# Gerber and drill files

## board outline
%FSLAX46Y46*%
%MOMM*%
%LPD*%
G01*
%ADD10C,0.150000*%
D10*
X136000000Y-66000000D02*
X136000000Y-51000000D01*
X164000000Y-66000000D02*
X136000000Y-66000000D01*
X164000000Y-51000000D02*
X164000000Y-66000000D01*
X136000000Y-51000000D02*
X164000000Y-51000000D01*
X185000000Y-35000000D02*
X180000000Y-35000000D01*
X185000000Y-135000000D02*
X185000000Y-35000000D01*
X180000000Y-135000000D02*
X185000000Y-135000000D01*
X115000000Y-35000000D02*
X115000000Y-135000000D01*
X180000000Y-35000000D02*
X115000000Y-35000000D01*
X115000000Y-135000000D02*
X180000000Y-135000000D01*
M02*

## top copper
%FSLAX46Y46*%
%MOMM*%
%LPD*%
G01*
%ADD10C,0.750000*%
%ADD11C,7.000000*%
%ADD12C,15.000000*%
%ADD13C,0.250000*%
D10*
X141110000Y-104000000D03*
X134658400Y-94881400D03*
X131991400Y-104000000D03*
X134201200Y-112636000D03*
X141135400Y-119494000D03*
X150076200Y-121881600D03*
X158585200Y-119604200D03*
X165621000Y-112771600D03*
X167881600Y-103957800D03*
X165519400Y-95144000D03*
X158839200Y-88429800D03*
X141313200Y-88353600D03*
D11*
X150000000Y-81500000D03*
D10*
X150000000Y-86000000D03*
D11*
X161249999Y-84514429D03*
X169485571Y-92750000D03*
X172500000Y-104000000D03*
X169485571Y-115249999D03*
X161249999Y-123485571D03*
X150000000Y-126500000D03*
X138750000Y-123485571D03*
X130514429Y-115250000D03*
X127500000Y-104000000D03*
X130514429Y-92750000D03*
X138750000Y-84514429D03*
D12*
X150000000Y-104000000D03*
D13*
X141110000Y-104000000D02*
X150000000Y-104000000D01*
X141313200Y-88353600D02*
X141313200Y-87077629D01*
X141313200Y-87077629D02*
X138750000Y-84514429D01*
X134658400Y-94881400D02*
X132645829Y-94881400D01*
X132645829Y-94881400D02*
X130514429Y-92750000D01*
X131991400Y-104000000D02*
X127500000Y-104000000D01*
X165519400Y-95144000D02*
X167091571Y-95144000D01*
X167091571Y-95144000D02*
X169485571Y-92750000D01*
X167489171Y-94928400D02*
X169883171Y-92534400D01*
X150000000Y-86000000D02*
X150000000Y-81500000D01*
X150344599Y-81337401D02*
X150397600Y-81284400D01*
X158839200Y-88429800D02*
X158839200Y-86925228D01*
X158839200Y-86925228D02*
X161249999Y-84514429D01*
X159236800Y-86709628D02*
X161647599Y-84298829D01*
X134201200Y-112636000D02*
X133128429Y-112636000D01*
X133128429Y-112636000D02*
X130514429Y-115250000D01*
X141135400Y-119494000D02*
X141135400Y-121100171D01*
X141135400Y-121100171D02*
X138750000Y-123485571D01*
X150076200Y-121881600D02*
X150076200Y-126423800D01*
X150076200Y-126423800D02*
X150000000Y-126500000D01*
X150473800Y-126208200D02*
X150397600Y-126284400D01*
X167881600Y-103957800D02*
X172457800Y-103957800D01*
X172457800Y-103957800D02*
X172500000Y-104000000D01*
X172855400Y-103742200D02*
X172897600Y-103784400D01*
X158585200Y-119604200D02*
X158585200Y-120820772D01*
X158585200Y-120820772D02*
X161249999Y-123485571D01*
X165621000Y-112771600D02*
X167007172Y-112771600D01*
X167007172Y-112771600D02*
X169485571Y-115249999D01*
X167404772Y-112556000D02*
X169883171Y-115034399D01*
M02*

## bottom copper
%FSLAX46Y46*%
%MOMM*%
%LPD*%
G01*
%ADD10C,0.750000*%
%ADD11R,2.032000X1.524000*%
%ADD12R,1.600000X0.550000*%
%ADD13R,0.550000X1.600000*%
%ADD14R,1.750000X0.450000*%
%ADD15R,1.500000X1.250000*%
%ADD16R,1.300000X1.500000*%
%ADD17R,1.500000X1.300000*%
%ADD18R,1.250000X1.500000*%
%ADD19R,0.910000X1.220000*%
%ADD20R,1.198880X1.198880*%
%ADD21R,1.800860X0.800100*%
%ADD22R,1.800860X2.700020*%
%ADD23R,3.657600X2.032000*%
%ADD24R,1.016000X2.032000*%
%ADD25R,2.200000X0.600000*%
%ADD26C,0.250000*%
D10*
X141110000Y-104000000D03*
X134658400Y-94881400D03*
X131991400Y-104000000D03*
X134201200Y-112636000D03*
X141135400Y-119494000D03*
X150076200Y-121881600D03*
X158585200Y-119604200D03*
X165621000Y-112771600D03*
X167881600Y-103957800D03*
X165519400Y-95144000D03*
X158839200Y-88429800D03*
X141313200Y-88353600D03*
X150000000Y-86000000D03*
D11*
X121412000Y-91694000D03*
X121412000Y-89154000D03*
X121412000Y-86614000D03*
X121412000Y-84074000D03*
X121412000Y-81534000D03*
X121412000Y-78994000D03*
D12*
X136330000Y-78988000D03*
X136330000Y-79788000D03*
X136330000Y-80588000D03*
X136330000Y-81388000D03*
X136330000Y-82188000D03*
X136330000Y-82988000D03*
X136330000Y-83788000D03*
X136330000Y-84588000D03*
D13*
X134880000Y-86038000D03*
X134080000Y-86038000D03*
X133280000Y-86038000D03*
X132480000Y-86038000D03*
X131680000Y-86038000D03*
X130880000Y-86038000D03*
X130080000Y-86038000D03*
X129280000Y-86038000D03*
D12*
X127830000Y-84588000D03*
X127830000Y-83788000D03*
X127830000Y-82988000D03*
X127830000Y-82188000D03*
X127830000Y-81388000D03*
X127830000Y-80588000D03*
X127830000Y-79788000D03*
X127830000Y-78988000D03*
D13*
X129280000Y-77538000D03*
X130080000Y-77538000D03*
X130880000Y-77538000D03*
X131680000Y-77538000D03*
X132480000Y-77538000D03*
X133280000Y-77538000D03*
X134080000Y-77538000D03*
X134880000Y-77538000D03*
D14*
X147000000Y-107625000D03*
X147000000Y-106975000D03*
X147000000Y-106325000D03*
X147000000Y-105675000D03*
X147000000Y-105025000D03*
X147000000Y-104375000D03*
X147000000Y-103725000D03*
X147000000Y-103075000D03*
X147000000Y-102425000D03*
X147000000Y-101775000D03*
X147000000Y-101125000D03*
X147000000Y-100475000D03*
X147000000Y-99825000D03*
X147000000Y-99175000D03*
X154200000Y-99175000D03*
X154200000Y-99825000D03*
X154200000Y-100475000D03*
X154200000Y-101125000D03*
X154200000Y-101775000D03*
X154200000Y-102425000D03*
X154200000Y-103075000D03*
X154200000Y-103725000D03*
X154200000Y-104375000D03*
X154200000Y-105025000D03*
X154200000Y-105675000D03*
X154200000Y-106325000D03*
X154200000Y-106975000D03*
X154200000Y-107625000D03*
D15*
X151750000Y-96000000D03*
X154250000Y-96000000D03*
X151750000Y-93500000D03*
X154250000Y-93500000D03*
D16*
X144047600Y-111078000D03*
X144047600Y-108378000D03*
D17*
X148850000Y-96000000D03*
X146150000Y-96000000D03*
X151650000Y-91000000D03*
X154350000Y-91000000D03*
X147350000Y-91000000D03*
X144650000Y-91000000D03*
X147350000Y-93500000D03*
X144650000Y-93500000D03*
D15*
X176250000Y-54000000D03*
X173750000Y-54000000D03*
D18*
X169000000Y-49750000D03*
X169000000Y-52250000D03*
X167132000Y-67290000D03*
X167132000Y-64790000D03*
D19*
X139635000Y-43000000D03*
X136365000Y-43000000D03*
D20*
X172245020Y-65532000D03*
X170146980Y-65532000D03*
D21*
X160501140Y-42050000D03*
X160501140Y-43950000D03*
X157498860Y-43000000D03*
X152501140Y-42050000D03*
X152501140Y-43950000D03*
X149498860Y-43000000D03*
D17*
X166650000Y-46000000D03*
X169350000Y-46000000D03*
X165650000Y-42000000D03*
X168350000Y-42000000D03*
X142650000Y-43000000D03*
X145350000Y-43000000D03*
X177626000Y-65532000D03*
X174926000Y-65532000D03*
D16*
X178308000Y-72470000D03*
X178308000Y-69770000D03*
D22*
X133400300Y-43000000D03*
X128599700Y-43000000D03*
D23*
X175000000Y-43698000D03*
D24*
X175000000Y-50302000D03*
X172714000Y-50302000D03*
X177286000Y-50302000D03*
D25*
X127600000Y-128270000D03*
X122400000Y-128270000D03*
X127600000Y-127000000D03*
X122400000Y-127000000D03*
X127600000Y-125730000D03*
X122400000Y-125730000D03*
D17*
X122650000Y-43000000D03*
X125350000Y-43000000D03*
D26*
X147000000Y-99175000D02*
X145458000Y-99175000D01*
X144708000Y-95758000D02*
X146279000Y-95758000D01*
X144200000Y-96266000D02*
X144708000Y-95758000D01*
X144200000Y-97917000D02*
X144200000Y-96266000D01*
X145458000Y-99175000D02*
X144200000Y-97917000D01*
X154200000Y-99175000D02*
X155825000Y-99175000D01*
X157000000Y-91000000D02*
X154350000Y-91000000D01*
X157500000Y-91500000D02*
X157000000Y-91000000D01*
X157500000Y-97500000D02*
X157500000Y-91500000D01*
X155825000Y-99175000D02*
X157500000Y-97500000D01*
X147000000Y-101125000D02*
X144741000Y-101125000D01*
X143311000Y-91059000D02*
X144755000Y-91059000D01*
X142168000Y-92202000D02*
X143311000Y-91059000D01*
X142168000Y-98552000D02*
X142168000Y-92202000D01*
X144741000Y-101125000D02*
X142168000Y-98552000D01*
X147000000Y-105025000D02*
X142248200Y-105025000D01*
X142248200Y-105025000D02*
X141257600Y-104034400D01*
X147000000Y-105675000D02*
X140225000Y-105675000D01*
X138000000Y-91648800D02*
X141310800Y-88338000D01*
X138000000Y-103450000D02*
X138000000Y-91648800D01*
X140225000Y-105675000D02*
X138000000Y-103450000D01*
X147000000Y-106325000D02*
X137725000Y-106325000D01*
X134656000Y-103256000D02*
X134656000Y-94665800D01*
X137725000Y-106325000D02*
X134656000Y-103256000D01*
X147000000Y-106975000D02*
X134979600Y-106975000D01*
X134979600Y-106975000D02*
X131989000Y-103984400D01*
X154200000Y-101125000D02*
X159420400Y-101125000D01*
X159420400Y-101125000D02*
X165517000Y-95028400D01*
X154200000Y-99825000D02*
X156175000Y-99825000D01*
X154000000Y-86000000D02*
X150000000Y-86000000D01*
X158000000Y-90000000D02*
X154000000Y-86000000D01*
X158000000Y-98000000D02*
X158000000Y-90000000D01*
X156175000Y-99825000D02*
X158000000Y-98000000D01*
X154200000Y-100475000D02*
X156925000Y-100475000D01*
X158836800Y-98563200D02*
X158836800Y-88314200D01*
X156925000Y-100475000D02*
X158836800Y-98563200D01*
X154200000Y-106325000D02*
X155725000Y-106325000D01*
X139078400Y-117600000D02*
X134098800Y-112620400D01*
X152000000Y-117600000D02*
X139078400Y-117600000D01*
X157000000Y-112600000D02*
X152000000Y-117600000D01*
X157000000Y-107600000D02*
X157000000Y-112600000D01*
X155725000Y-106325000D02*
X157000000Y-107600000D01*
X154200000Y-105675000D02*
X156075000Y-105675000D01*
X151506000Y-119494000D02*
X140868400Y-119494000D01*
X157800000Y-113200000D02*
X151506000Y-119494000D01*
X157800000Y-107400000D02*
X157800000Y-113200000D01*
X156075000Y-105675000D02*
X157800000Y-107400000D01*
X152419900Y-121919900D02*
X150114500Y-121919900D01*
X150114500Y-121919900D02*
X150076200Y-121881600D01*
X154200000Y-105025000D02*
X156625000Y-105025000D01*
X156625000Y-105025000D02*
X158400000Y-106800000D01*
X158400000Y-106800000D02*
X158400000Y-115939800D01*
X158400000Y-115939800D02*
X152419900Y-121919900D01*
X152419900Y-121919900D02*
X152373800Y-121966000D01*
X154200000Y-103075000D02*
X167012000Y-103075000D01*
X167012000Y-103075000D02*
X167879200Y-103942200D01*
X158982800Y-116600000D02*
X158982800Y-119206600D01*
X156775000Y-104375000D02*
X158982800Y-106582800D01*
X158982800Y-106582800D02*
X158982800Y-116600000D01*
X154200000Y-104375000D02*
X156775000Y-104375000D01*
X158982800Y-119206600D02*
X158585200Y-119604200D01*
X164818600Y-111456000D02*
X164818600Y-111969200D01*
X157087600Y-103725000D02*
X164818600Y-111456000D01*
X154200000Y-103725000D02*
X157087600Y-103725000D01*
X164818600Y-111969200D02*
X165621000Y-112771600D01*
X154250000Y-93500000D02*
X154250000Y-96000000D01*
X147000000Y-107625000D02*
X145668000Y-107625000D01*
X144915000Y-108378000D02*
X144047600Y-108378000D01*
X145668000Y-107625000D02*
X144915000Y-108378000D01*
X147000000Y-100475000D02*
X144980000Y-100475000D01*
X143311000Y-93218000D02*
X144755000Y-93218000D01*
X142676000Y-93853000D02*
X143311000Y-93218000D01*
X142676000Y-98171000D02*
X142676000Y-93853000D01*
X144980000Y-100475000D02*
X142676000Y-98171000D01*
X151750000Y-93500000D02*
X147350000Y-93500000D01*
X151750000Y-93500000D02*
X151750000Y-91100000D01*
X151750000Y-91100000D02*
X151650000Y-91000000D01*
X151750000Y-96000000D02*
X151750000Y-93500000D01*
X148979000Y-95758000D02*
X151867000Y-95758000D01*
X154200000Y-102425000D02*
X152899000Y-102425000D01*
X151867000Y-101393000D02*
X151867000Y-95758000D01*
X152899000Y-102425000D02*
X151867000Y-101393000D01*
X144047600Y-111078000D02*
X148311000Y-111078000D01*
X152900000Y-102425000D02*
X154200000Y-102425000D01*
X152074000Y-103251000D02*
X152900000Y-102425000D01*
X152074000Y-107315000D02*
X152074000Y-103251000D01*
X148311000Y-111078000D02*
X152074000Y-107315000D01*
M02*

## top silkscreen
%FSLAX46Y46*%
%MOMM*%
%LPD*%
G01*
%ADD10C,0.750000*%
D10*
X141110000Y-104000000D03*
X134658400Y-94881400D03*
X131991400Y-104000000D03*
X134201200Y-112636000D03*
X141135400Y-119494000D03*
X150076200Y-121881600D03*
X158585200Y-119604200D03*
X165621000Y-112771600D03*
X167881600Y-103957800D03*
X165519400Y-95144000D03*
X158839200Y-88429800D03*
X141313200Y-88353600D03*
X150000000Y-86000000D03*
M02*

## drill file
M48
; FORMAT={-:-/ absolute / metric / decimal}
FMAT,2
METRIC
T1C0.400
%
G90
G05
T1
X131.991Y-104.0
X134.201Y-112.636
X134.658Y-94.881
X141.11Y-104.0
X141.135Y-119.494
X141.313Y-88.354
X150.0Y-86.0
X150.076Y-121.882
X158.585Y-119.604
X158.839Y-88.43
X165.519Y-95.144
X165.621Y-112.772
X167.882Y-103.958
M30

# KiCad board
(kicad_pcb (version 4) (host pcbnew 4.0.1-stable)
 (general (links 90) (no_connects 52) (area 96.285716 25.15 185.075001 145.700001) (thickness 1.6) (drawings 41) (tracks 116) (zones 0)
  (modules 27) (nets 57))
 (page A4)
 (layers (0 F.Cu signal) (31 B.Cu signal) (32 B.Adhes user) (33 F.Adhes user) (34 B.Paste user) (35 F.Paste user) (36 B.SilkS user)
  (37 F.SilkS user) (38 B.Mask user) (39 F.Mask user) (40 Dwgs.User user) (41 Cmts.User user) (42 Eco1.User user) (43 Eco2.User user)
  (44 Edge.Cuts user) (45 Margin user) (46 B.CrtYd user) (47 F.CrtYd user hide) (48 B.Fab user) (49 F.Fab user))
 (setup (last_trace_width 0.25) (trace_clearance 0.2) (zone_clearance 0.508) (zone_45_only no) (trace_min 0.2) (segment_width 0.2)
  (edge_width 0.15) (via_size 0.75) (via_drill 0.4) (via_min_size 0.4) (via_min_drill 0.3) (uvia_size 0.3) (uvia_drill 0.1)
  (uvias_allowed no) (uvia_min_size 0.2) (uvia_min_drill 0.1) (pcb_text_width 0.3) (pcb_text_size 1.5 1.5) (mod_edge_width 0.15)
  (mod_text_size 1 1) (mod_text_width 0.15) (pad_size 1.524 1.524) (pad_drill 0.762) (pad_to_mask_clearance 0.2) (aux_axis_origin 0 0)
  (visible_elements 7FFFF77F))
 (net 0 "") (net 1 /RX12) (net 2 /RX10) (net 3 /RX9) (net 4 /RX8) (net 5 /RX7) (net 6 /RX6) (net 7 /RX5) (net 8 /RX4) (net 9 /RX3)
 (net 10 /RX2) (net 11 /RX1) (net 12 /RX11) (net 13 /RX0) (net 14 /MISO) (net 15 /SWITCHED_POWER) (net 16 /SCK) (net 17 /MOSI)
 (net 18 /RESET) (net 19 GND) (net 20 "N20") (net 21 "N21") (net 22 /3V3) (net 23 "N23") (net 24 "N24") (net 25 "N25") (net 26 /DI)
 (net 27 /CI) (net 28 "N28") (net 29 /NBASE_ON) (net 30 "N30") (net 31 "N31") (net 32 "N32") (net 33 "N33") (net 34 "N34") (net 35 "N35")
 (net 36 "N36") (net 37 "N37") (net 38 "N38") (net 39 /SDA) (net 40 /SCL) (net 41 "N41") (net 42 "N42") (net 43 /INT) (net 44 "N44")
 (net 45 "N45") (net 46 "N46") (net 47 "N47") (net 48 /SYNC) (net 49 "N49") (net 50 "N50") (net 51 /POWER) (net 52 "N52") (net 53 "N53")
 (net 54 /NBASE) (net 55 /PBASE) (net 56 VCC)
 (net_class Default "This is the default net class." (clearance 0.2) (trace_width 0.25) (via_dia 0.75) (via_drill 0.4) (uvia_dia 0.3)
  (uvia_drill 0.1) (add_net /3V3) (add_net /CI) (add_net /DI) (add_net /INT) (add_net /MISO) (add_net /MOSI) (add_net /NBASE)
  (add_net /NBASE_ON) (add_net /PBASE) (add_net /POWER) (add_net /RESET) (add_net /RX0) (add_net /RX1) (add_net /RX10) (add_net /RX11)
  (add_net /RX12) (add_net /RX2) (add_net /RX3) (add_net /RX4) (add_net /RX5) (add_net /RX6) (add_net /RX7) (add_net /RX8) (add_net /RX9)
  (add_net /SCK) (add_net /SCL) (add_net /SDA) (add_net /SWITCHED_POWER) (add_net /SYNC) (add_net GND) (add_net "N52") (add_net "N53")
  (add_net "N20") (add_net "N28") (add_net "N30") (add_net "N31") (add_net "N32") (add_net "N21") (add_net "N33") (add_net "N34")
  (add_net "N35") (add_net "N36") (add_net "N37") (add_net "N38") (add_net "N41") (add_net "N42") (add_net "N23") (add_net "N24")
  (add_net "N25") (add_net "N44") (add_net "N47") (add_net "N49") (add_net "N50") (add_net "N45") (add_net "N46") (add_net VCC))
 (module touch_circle (layer F.Cu) (at 150 104)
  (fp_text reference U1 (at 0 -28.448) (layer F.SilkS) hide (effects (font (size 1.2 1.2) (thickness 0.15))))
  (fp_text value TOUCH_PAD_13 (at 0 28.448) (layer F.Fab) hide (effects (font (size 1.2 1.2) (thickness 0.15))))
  (pad 13 thru_hole circle (at -8.89 0) (size 0.75 0.75) (drill 0.4) (layers *.Cu *.Mask F.SilkS) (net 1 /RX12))
  (pad 11 thru_hole circle (at -15.3416 -9.1186) (size 0.75 0.75) (drill 0.4) (layers *.Cu *.Mask F.SilkS) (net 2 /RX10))
  (pad 10 thru_hole circle (at -18.0086 0) (size 0.75 0.75) (drill 0.4) (layers *.Cu *.Mask F.SilkS) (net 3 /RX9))
  (pad 9 thru_hole circle (at -15.7988 8.636) (size 0.75 0.75) (drill 0.4) (layers *.Cu *.Mask F.SilkS) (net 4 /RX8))
  (pad 8 thru_hole circle (at -8.8646 15.494) (size 0.75 0.75) (drill 0.4) (layers *.Cu *.Mask F.SilkS) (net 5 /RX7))
  (pad 7 thru_hole circle (at 0.0762 17.8816) (size 0.75 0.75) (drill 0.4) (layers *.Cu *.Mask F.SilkS) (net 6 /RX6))
  (pad 6 thru_hole circle (at 8.5852 15.6042) (size 0.75 0.75) (drill 0.4) (layers *.Cu *.Mask F.SilkS) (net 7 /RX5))
  (pad 5 thru_hole circle (at 15.621 8.7716) (size 0.75 0.75) (drill 0.4) (layers *.Cu *.Mask F.SilkS) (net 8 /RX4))
  (pad 4 thru_hole circle (at 17.8816 -0.0422) (size 0.75 0.75) (drill 0.4) (layers *.Cu *.Mask F.SilkS) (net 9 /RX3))
  (pad 3 thru_hole circle (at 15.5194 -8.856) (size 0.75 0.75) (drill 0.4) (layers *.Cu *.Mask F.SilkS) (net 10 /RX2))
  (pad 2 thru_hole circle (at 8.8392 -15.5702) (size 0.75 0.75) (drill 0.4) (layers *.Cu *.Mask F.SilkS) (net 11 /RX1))
  (pad 12 thru_hole circle (at -8.6868 -15.6464) (size 0.75 0.75) (drill 0.4) (layers *.Cu *.Mask F.SilkS) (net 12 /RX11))
  (pad 1 smd circle (at 0 -22.5) (size 7 7) (layers F.Cu) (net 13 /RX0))
  (pad 1 thru_hole circle (at 0 -18) (size 0.75 0.75) (drill 0.4) (layers *.Cu *.Mask F.SilkS) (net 13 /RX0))
  (pad 2 smd circle (at 11.249999 -19.485571) (size 7 7) (layers F.Cu) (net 11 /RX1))
  (pad 3 smd circle (at 19.485571 -11.25) (size 7 7) (layers F.Cu) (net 10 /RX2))
  (pad 4 smd circle (at 22.5 0) (size 7 7) (layers F.Cu) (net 9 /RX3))
  (pad 5 smd circle (at 19.485571 11.249999) (size 7 7) (layers F.Cu) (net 8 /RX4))
  (pad 6 smd circle (at 11.249999 19.485571) (size 7 7) (layers F.Cu) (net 7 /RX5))
  (pad 7 smd circle (at 0 22.5) (size 7 7) (layers F.Cu) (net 6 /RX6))
  (pad 8 smd circle (at -11.25 19.485571) (size 7 7) (layers F.Cu) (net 5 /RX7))
  (pad 9 smd circle (at -19.485571 11.25) (size 7 7) (layers F.Cu) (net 4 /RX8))
  (pad 10 smd circle (at -22.5 0) (size 7 7) (layers F.Cu) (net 3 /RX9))
  (pad 11 smd circle (at -19.485571 -11.25) (size 7 7) (layers F.Cu) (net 2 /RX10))
  (pad 12 smd circle (at -11.25 -19.485571) (size 7 7) (layers F.Cu) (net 12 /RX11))
  (pad 13 smd circle (at 0 0) (size 15 15) (layers F.Cu) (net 1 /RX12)))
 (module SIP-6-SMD (layer B.Cu) (at 121.412 85.344 90)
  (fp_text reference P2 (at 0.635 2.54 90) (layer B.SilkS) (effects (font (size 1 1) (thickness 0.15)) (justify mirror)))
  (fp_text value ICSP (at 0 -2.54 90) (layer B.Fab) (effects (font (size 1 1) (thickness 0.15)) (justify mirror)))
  (pad 1 smd rect (at -6.35 0 90) (size 1.524 2.032) (layers B.Cu B.Paste B.Mask) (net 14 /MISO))
  (pad 2 smd rect (at -3.81 0 90) (size 1.524 2.032) (layers B.Cu B.Paste B.Mask) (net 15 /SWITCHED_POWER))
  (pad 3 smd rect (at -1.27 0 90) (size 1.524 2.032) (layers B.Cu B.Paste B.Mask) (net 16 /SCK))
  (pad 4 smd rect (at 1.27 0 90) (size 1.524 2.032) (layers B.Cu B.Paste B.Mask) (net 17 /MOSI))
  (pad 5 smd rect (at 3.81 0 90) (size 1.524 2.032) (layers B.Cu B.Paste B.Mask) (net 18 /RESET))
  (pad 6 smd rect (at 6.35 0 90) (size 1.524 2.032) (layers B.Cu B.Paste B.Mask) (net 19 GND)))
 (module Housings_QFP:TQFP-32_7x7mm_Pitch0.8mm (layer B.Cu) (at 132.08 81.788 180)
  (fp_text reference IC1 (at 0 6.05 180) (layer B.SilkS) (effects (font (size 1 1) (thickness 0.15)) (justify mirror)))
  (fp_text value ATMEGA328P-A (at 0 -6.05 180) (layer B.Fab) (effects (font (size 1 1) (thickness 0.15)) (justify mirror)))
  (pad 1 smd rect (at -4.25 2.8 180) (size 1.6 0.55) (layers B.Cu B.Paste B.Mask) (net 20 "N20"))
  (pad 2 smd rect (at -4.25 2 180) (size 1.6 0.55) (layers B.Cu B.Paste B.Mask) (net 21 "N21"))
  (pad 3 smd rect (at -4.25 1.2 180) (size 1.6 0.55) (layers B.Cu B.Paste B.Mask) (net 19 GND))
  (pad 4 smd rect (at -4.25 0.4 180) (size 1.6 0.55) (layers B.Cu B.Paste B.Mask) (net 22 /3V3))
  (pad 5 smd rect (at -4.25 -0.4 180) (size 1.6 0.55) (layers B.Cu B.Paste B.Mask) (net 19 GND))
  (pad 6 smd rect (at -4.25 -1.2 180) (size 1.6 0.55) (layers B.Cu B.Paste B.Mask) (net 22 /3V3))
  (pad 7 smd rect (at -4.25 -2 180) (size 1.6 0.55) (layers B.Cu B.Paste B.Mask) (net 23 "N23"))
  (pad 8 smd rect (at -4.25 -2.8 180) (size 1.6 0.55) (layers B.Cu B.Paste B.Mask) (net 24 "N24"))
  (pad 9 smd rect (at -2.8 -4.25 90) (size 1.6 0.55) (layers B.Cu B.Paste B.Mask) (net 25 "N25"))
  (pad 10 smd rect (at -2 -4.25 90) (size 1.6 0.55) (layers B.Cu B.Paste B.Mask) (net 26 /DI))
  (pad 11 smd rect (at -1.2 -4.25 90) (size 1.6 0.55) (layers B.Cu B.Paste B.Mask) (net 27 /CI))
  (pad 12 smd rect (at -0.4 -4.25 90) (size 1.6 0.55) (layers B.Cu B.Paste B.Mask) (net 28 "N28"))
  (pad 13 smd rect (at 0.4 -4.25 90) (size 1.6 0.55) (layers B.Cu B.Paste B.Mask) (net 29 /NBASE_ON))
  (pad 14 smd rect (at 1.2 -4.25 90) (size 1.6 0.55) (layers B.Cu B.Paste B.Mask) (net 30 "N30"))
  (pad 15 smd rect (at 2 -4.25 90) (size 1.6 0.55) (layers B.Cu B.Paste B.Mask) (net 17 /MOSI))
  (pad 16 smd rect (at 2.8 -4.25 90) (size 1.6 0.55) (layers B.Cu B.Paste B.Mask) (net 14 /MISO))
  (pad 17 smd rect (at 4.25 -2.8 180) (size 1.6 0.55) (layers B.Cu B.Paste B.Mask) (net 16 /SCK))
  (pad 18 smd rect (at 4.25 -2 180) (size 1.6 0.55) (layers B.Cu B.Paste B.Mask) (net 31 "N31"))
  (pad 19 smd rect (at 4.25 -1.2 180) (size 1.6 0.55) (layers B.Cu B.Paste B.Mask) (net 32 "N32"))
  (pad 20 smd rect (at 4.25 -0.4 180) (size 1.6 0.55) (layers B.Cu B.Paste B.Mask) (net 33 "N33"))
  (pad 21 smd rect (at 4.25 0.4 180) (size 1.6 0.55) (layers B.Cu B.Paste B.Mask) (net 19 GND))
  (pad 22 smd rect (at 4.25 1.2 180) (size 1.6 0.55) (layers B.Cu B.Paste B.Mask) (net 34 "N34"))
  (pad 23 smd rect (at 4.25 2 180) (size 1.6 0.55) (layers B.Cu B.Paste B.Mask) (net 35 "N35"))
  (pad 24 smd rect (at 4.25 2.8 180) (size 1.6 0.55) (layers B.Cu B.Paste B.Mask) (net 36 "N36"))
  (pad 25 smd rect (at 2.8 4.25 90) (size 1.6 0.55) (layers B.Cu B.Paste B.Mask) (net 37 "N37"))
  (pad 26 smd rect (at 2 4.25 90) (size 1.6 0.55) (layers B.Cu B.Paste B.Mask) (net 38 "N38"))
  (pad 27 smd rect (at 1.2 4.25 90) (size 1.6 0.55) (layers B.Cu B.Paste B.Mask) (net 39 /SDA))
  (pad 28 smd rect (at 0.4 4.25 90) (size 1.6 0.55) (layers B.Cu B.Paste B.Mask) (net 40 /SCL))
  (pad 29 smd rect (at -0.4 4.25 90) (size 1.6 0.55) (layers B.Cu B.Paste B.Mask) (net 18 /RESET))
  (pad 30 smd rect (at -1.2 4.25 90) (size 1.6 0.55) (layers B.Cu B.Paste B.Mask) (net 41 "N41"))
  (pad 31 smd rect (at -2 4.25 90) (size 1.6 0.55) (layers B.Cu B.Paste B.Mask) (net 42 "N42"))
  (pad 32 smd rect (at -2.8 4.25 90) (size 1.6 0.55) (layers B.Cu B.Paste B.Mask) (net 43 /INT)))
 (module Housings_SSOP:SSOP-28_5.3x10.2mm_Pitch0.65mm (layer B.Cu) (at 150.6 103.4)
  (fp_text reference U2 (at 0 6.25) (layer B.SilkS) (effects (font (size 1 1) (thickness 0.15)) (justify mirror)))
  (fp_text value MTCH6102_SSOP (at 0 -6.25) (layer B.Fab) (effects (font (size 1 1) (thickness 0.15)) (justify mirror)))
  (pad 1 smd rect (at -3.6 4.225) (size 1.75 0.45) (layers B.Cu B.Paste B.Mask) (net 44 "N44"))
  (pad 2 smd rect (at -3.6 3.575) (size 1.75 0.45) (layers B.Cu B.Paste B.Mask) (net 3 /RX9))
  (pad 3 smd rect (at -3.6 2.925) (size 1.75 0.45) (layers B.Cu B.Paste B.Mask) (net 2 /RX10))
  (pad 4 smd rect (at -3.6 2.275) (size 1.75 0.45) (layers B.Cu B.Paste B.Mask) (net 12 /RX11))
  (pad 5 smd rect (at -3.6 1.625) (size 1.75 0.45) (layers B.Cu B.Paste B.Mask) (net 1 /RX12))
  (pad 6 smd rect (at -3.6 0.975) (size 1.75 0.45) (layers B.Cu B.Paste B.Mask) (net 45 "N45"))
  (pad 7 smd rect (at -3.6 0.325) (size 1.75 0.45) (layers B.Cu B.Paste B.Mask) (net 19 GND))
  (pad 8 smd rect (at -3.6 -0.325) (size 1.75 0.45) (layers B.Cu B.Paste B.Mask) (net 19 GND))
  (pad 9 smd rect (at -3.6 -0.975) (size 1.75 0.45) (layers B.Cu B.Paste B.Mask) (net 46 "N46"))
  (pad 10 smd rect (at -3.6 -1.625) (size 1.75 0.45) (layers B.Cu B.Paste B.Mask) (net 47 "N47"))
  (pad 11 smd rect (at -3.6 -2.275) (size 1.75 0.45) (layers B.Cu B.Paste B.Mask) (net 43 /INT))
  (pad 12 smd rect (at -3.6 -2.925) (size 1.75 0.45) (layers B.Cu B.Paste B.Mask) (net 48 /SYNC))
  (pad 13 smd rect (at -3.6 -3.575) (size 1.75 0.45) (layers B.Cu B.Paste B.Mask) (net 19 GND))
  (pad 14 smd rect (at -3.6 -4.225) (size 1.75 0.45) (layers B.Cu B.Paste B.Mask) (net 39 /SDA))
  (pad 15 smd rect (at 3.6 -4.225) (size 1.75 0.45) (layers B.Cu B.Paste B.Mask) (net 40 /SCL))
  (pad 16 smd rect (at 3.6 -3.575) (size 1.75 0.45) (layers B.Cu B.Paste B.Mask) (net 13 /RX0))
  (pad 17 smd rect (at 3.6 -2.925) (size 1.75 0.45) (layers B.Cu B.Paste B.Mask) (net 11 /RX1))
  (pad 18 smd rect (at 3.6 -2.275) (size 1.75 0.45) (layers B.Cu B.Paste B.Mask) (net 10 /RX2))
  (pad 19 smd rect (at 3.6 -1.625) (size 1.75 0.45) (layers B.Cu B.Paste B.Mask) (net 19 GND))
  (pad 20 smd rect (at 3.6 -0.975) (size 1.75 0.45) (layers B.Cu B.Paste B.Mask) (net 22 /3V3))
  (pad 21 smd rect (at 3.6 -0.325) (size 1.75 0.45) (layers B.Cu B.Paste B.Mask) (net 9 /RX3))
  (pad 22 smd rect (at 3.6 0.325) (size 1.75 0.45) (layers B.Cu B.Paste B.Mask) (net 8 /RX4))
  (pad 23 smd rect (at 3.6 0.975) (size 1.75 0.45) (layers B.Cu B.Paste B.Mask) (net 7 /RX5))
  (pad 24 smd rect (at 3.6 1.625) (size 1.75 0.45) (layers B.Cu B.Paste B.Mask) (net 6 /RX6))
  (pad 25 smd rect (at 3.6 2.275) (size 1.75 0.45) (layers B.Cu B.Paste B.Mask) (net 5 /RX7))
  (pad 26 smd rect (at 3.6 2.925) (size 1.75 0.45) (layers B.Cu B.Paste B.Mask) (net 4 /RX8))
  (pad 27 smd rect (at 3.6 3.575) (size 1.75 0.45) (layers B.Cu B.Paste B.Mask) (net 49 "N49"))
  (pad 28 smd rect (at 3.6 4.225) (size 1.75 0.45) (layers B.Cu B.Paste B.Mask) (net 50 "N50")))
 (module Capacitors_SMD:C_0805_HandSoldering (layer B.Cu) (at 153 96)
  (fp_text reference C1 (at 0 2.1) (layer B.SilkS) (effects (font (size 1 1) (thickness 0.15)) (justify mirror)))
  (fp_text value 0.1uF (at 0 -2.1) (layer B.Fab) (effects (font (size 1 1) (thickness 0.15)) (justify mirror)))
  (pad 1 smd rect (at -1.25 0) (size 1.5 1.25) (layers B.Cu B.Paste B.Mask) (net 22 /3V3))
  (pad 2 smd rect (at 1.25 0) (size 1.5 1.25) (layers B.Cu B.Paste B.Mask) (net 19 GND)))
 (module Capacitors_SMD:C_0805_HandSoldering (layer B.Cu) (at 153 93.5)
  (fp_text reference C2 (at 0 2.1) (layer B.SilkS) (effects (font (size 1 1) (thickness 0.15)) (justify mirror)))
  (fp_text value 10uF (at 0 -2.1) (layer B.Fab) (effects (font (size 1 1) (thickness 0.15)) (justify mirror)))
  (pad 1 smd rect (at -1.25 0) (size 1.5 1.25) (layers B.Cu B.Paste B.Mask) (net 22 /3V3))
  (pad 2 smd rect (at 1.25 0) (size 1.5 1.25) (layers B.Cu B.Paste B.Mask) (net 19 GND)))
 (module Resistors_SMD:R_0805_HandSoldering (layer B.Cu) (at 144.0476 109.728 90)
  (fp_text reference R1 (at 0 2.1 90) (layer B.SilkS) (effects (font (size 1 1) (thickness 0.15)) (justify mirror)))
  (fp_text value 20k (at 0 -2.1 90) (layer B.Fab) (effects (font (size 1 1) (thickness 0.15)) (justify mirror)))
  (pad 1 smd rect (at -1.35 0 90) (size 1.5 1.3) (layers B.Cu B.Paste B.Mask) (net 22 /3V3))
  (pad 2 smd rect (at 1.35 0 90) (size 1.5 1.3) (layers B.Cu B.Paste B.Mask) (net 44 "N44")))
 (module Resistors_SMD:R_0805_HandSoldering (layer B.Cu) (at 147.5 96 180)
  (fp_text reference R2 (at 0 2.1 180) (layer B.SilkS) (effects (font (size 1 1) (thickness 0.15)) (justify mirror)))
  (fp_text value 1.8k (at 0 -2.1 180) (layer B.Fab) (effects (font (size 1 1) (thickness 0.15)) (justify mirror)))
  (pad 1 smd rect (at -1.35 0 180) (size 1.5 1.3) (layers B.Cu B.Paste B.Mask) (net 22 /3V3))
  (pad 2 smd rect (at 1.35 0 180) (size 1.5 1.3) (layers B.Cu B.Paste B.Mask) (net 39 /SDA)))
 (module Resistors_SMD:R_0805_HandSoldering (layer B.Cu) (at 153 91)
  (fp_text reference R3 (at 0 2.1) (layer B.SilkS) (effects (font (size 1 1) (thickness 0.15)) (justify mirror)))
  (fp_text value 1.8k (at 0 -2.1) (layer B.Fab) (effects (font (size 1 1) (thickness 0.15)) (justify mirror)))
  (pad 1 smd rect (at -1.35 0) (size 1.5 1.3) (layers B.Cu B.Paste B.Mask) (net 22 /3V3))
  (pad 2 smd rect (at 1.35 0) (size 1.5 1.3) (layers B.Cu B.Paste B.Mask) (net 40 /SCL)))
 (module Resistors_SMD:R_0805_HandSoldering (layer B.Cu) (at 146 91 180)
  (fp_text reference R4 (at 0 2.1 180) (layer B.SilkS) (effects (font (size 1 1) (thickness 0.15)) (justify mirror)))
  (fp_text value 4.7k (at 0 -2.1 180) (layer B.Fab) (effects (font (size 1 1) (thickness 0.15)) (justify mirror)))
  (pad 1 smd rect (at -1.35 0 180) (size 1.5 1.3) (layers B.Cu B.Paste B.Mask) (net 22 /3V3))
  (pad 2 smd rect (at 1.35 0 180) (size 1.5 1.3) (layers B.Cu B.Paste B.Mask) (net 43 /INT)))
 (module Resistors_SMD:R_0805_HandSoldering (layer B.Cu) (at 146 93.5 180)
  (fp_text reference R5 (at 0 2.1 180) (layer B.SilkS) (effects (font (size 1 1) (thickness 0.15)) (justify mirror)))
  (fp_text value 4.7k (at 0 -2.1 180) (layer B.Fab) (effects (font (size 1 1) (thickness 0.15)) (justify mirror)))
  (pad 1 smd rect (at -1.35 0 180) (size 1.5 1.3) (layers B.Cu B.Paste B.Mask) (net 22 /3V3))
  (pad 2 smd rect (at 1.35 0 180) (size 1.5 1.3) (layers B.Cu B.Paste B.Mask) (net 48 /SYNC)))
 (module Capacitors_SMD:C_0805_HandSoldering (layer B.Cu) (at 175 54 180)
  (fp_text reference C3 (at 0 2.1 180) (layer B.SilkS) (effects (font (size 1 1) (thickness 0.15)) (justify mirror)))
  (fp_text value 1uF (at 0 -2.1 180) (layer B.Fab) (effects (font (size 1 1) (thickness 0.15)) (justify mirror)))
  (pad 1 smd rect (at -1.25 0 180) (size 1.5 1.25) (layers B.Cu B.Paste B.Mask) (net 15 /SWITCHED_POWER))
  (pad 2 smd rect (at 1.25 0 180) (size 1.5 1.25) (layers B.Cu B.Paste B.Mask) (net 19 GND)))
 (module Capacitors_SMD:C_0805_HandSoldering (layer B.Cu) (at 169 51 270)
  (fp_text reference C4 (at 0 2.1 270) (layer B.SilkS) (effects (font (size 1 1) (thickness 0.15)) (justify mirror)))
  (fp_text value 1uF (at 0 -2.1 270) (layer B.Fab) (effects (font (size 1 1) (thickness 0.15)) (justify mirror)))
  (pad 1 smd rect (at -1.25 0 270) (size 1.5 1.25) (layers B.Cu B.Paste B.Mask) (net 22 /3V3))
  (pad 2 smd rect (at 1.25 0 270) (size 1.5 1.25) (layers B.Cu B.Paste B.Mask) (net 19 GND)))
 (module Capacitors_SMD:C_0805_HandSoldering (layer B.Cu) (at 167.132 66.04 90)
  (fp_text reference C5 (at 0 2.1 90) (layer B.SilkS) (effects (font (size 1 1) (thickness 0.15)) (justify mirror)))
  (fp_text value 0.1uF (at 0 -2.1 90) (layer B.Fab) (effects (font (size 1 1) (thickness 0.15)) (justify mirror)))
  (pad 1 smd rect (at -1.25 0 90) (size 1.5 1.25) (layers B.Cu B.Paste B.Mask) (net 22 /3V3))
  (pad 2 smd rect (at 1.25 0 90) (size 1.5 1.25) (layers B.Cu B.Paste B.Mask) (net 19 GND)))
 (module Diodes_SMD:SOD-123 (layer B.Cu) (at 138 43 180)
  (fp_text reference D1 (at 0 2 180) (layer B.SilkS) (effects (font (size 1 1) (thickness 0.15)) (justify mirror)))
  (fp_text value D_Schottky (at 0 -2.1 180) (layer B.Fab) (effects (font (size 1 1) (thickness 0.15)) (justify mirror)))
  (pad 1 smd rect (at -1.635 0 180) (size 0.91 1.22) (layers B.Cu B.Paste B.Mask) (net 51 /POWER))
  (pad 2 smd rect (at 1.635 0 180) (size 0.91 1.22) (layers B.Cu B.Paste B.Mask) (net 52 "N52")))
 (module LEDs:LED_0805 (layer B.Cu) (at 171.196 65.532)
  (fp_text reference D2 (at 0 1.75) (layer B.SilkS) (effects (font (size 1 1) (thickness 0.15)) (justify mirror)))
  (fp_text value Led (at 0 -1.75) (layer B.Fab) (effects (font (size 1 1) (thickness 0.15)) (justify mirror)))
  (pad 2 smd rect (at 1.04902 0 180) (size 1.19888 1.19888) (layers B.Cu B.Paste B.Mask) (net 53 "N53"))
  (pad 1 smd rect (at -1.04902 0 180) (size 1.19888 1.19888) (layers B.Cu B.Paste B.Mask) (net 19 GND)))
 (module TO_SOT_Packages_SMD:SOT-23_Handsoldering (layer B.Cu) (at 159 43 270)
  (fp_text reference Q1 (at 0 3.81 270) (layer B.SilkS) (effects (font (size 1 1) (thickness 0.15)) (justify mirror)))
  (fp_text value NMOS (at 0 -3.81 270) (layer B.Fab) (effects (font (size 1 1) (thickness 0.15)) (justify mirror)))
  (pad 1 smd rect (at -0.95 -1.50114 270) (size 0.8001 1.80086) (layers B.Cu B.Paste B.Mask) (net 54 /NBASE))
  (pad 2 smd rect (at 0.95 -1.50114 270) (size 0.8001 1.80086) (layers B.Cu B.Paste B.Mask) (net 19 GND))
  (pad 3 smd rect (at 0 1.50114 270) (size 0.8001 1.80086) (layers B.Cu B.Paste B.Mask) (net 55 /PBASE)))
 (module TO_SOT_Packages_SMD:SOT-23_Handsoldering (layer B.Cu) (at 151 43 270)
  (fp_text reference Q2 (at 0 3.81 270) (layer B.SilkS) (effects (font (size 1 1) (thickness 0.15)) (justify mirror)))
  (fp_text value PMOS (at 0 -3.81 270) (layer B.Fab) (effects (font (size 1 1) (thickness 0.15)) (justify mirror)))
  (pad 1 smd rect (at -0.95 -1.50114 270) (size 0.8001 1.80086) (layers B.Cu B.Paste B.Mask) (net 55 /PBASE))
  (pad 2 smd rect (at 0.95 -1.50114 270) (size 0.8001 1.80086) (layers B.Cu B.Paste B.Mask) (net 15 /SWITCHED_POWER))
  (pad 3 smd rect (at 0 1.50114 270) (size 0.8001 1.80086) (layers B.Cu B.Paste B.Mask) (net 51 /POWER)))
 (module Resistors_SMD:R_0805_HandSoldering (layer B.Cu) (at 168 46)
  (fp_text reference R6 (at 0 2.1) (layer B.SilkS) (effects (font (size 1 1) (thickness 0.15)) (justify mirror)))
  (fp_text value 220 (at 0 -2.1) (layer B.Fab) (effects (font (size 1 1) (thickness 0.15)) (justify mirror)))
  (pad 1 smd rect (at -1.35 0) (size 1.5 1.3) (layers B.Cu B.Paste B.Mask) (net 54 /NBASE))
  (pad 2 smd rect (at 1.35 0) (size 1.5 1.3) (layers B.Cu B.Paste B.Mask) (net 29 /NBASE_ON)))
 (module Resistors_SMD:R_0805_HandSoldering (layer B.Cu) (at 167 42)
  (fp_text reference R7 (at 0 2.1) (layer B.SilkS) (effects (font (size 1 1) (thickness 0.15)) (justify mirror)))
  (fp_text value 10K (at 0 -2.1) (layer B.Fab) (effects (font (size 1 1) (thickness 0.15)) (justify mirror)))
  (pad 1 smd rect (at -1.35 0) (size 1.5 1.3) (layers B.Cu B.Paste B.Mask) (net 54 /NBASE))
  (pad 2 smd rect (at 1.35 0) (size 1.5 1.3) (layers B.Cu B.Paste B.Mask) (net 19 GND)))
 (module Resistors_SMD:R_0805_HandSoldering (layer B.Cu) (at 144 43)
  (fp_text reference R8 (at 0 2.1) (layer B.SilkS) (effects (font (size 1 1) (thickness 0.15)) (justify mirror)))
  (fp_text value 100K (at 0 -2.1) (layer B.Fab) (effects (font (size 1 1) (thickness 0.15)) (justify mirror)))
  (pad 1 smd rect (at -1.35 0) (size 1.5 1.3) (layers B.Cu B.Paste B.Mask) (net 51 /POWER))
  (pad 2 smd rect (at 1.35 0) (size 1.5 1.3) (layers B.Cu B.Paste B.Mask) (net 55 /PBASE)))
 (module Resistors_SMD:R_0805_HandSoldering (layer B.Cu) (at 176.276 65.532 180)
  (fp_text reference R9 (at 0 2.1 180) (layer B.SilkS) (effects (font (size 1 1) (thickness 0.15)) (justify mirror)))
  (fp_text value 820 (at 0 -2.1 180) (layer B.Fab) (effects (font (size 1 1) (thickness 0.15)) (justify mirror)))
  (pad 1 smd rect (at -1.35 0 180) (size 1.5 1.3) (layers B.Cu B.Paste B.Mask) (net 16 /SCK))
  (pad 2 smd rect (at 1.35 0 180) (size 1.5 1.3) (layers B.Cu B.Paste B.Mask) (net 53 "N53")))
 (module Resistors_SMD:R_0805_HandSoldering (layer B.Cu) (at 178.308 71.12 90)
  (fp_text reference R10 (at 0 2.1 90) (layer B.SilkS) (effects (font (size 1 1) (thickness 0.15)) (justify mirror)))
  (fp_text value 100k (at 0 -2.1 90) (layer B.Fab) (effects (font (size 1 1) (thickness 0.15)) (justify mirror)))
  (pad 1 smd rect (at -1.35 0 90) (size 1.5 1.3) (layers B.Cu B.Paste B.Mask) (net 18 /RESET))
  (pad 2 smd rect (at 1.35 0 90) (size 1.5 1.3) (layers B.Cu B.Paste B.Mask) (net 19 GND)))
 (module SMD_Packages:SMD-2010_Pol (layer B.Cu) (at 131 43 180)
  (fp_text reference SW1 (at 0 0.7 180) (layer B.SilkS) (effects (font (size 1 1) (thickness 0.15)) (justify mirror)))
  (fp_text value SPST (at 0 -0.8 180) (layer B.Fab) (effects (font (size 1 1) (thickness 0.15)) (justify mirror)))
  (pad 1 smd rect (at -2.4003 0 180) (size 1.80086 2.70002) (layers B.Cu B.Paste B.Mask) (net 52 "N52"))
  (pad 2 smd rect (at 2.4003 0 180) (size 1.80086 2.70002) (layers B.Cu B.Paste B.Mask) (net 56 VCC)))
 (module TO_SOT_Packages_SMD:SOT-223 (layer B.Cu) (at 175 47 180)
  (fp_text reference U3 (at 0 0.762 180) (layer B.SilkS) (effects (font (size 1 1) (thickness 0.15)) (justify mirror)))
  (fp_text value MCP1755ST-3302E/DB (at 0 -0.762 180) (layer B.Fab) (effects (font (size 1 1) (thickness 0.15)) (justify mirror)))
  (pad 4 smd rect (at 0 3.302 180) (size 3.6576 2.032) (layers B.Cu B.Paste B.Mask) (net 19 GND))
  (pad 2 smd rect (at 0 -3.302 180) (size 1.016 2.032) (layers B.Cu B.Paste B.Mask) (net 19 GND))
  (pad 3 smd rect (at 2.286 -3.302 180) (size 1.016 2.032) (layers B.Cu B.Paste B.Mask) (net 22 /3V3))
  (pad 1 smd rect (at -2.286 -3.302 180) (size 1.016 2.032) (layers B.Cu B.Paste B.Mask) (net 15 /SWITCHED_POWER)))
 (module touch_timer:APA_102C (layer B.Cu) (at 125 127 90)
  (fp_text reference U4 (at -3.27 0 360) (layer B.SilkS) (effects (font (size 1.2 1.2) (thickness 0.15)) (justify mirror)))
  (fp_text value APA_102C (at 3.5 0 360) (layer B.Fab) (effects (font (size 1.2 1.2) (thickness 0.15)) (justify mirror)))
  (pad 6 smd rect (at -1.27 2.6 90) (size 0.6 2.2) (layers B.Cu B.Paste B.Mask) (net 19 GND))
  (pad 1 smd rect (at -1.27 -2.6 90) (size 0.6 2.2) (layers B.Cu B.Paste B.Mask) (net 26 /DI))
  (pad 5 smd rect (at 0 2.6 90) (size 0.6 2.2) (layers B.Cu B.Paste B.Mask) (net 19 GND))
  (pad 2 smd rect (at 0 -2.6 90) (size 0.6 2.2) (layers B.Cu B.Paste B.Mask) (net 27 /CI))
  (pad 4 smd rect (at 1.27 2.6 90) (size 0.6 2.2) (layers B.Cu B.Paste B.Mask) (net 51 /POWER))
  (pad 3 smd rect (at 1.27 -2.6 90) (size 0.6 2.2) (layers B.Cu B.Paste B.Mask) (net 19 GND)))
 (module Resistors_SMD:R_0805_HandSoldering (layer B.Cu) (at 124 43)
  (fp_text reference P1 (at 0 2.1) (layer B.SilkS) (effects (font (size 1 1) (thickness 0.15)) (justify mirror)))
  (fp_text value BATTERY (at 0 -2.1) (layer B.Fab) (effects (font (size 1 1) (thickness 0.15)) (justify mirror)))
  (pad 1 smd rect (at -1.35 0) (size 1.5 1.3) (layers B.Cu B.Paste B.Mask) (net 19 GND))
  (pad 2 smd rect (at 1.35 0) (size 1.5 1.3) (layers B.Cu B.Paste B.Mask) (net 56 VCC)))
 (gr_line (start 136 66) (end 136 51) (angle 90) (layer Edge.Cuts) (width 0.15))
 (gr_line (start 164 66) (end 136 66) (angle 90) (layer Edge.Cuts) (width 0.15))
 (gr_line (start 164 51) (end 164 66) (angle 90) (layer Edge.Cuts) (width 0.15))
 (gr_line (start 136 51) (end 164 51) (angle 90) (layer Edge.Cuts) (width 0.15))
 (gr_line (start 185 35) (end 180 35) (angle 90) (layer Edge.Cuts) (width 0.15))
 (gr_line (start 185 135) (end 185 35) (angle 90) (layer Edge.Cuts) (width 0.15))
 (gr_line (start 180 135) (end 185 135) (angle 90) (layer Edge.Cuts) (width 0.15))
 (gr_line (start 115 35) (end 115 135) (angle 90) (layer Edge.Cuts) (width 0.15))
 (gr_line (start 180 35) (end 115 35) (angle 90) (layer Edge.Cuts) (width 0.15))
 (gr_line (start 115 135) (end 180 135) (angle 90) (layer Edge.Cuts) (width 0.15))
 (segment (start 147 99.175) (end 145.458 99.175) (width 0.25) (layer B.Cu) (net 39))
 (segment (start 144.708 95.758) (end 146.279 95.758) (width 0.25) (layer B.Cu) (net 39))
 (segment (start 144.2 96.266) (end 144.708 95.758) (width 0.25) (layer B.Cu) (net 39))
 (segment (start 144.2 97.917) (end 144.2 96.266) (width 0.25) (layer B.Cu) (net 39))
 (segment (start 145.458 99.175) (end 144.2 97.917) (width 0.25) (layer B.Cu) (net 39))
 (segment (start 154.2 99.175) (end 155.825 99.175) (width 0.25) (layer B.Cu) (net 40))
 (segment (start 157 91) (end 154.35 91) (width 0.25) (layer B.Cu) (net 40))
 (segment (start 157.5 91.5) (end 157 91) (width 0.25) (layer B.Cu) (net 40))
 (segment (start 157.5 97.5) (end 157.5 91.5) (width 0.25) (layer B.Cu) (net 40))
 (segment (start 155.825 99.175) (end 157.5 97.5) (width 0.25) (layer B.Cu) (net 40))
 (segment (start 147 101.125) (end 144.741 101.125) (width 0.25) (layer B.Cu) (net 43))
 (segment (start 143.311 91.059) (end 144.755 91.059) (width 0.25) (layer B.Cu) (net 43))
 (segment (start 142.168 92.202) (end 143.311 91.059) (width 0.25) (layer B.Cu) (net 43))
 (segment (start 142.168 98.552) (end 142.168 92.202) (width 0.25) (layer B.Cu) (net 43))
 (segment (start 144.741 101.125) (end 142.168 98.552) (width 0.25) (layer B.Cu) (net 43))
 (segment (start 141.11 104) (end 150 104) (width 0.25) (layer F.Cu) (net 1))
 (segment (start 147 105.025) (end 142.2482 105.025) (width 0.25) (layer B.Cu) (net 1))
 (segment (start 142.2482 105.025) (end 141.2576 104.0344) (width 0.25) (layer B.Cu) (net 1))
 (segment (start 141.3132 88.3536) (end 141.3132 87.077629) (width 0.25) (layer F.Cu) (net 12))
 (segment (start 141.3132 87.077629) (end 138.75 84.514429) (width 0.25) (layer F.Cu) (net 12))
 (segment (start 147 105.675) (end 140.225 105.675) (width 0.25) (layer B.Cu) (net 12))
 (segment (start 138 91.6488) (end 141.3108 88.338) (width 0.25) (layer B.Cu) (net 12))
 (segment (start 138 103.45) (end 138 91.6488) (width 0.25) (layer B.Cu) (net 12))
 (segment (start 140.225 105.675) (end 138 103.45) (width 0.25) (layer B.Cu) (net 12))
 (segment (start 134.6584 94.8814) (end 132.645829 94.8814) (width 0.25) (layer F.Cu) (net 2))
 (segment (start 132.645829 94.8814) (end 130.514429 92.75) (width 0.25) (layer F.Cu) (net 2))
 (segment (start 147 106.325) (end 137.725 106.325) (width 0.25) (layer B.Cu) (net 2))
 (segment (start 134.656 103.256) (end 134.656 94.6658) (width 0.25) (layer B.Cu) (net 2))
 (segment (start 137.725 106.325) (end 134.656 103.256) (width 0.25) (layer B.Cu) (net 2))
 (segment (start 131.9914 104) (end 127.5 104) (width 0.25) (layer F.Cu) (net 3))
 (segment (start 147 106.975) (end 134.9796 106.975) (width 0.25) (layer B.Cu) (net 3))
 (segment (start 134.9796 106.975) (end 131.989 103.9844) (width 0.25) (layer B.Cu) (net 3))
 (segment (start 165.5194 95.144) (end 167.091571 95.144) (width 0.25) (layer F.Cu) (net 10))
 (segment (start 167.091571 95.144) (end 169.485571 92.75) (width 0.25) (layer F.Cu) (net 10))
 (segment (start 167.489171 94.9284) (end 169.883171 92.5344) (width 0.25) (layer F.Cu) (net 10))
 (segment (start 154.2 101.125) (end 159.4204 101.125) (width 0.25) (layer B.Cu) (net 10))
 (segment (start 159.4204 101.125) (end 165.517 95.0284) (width 0.25) (layer B.Cu) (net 10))
 (segment (start 154.2 99.825) (end 156.175 99.825) (width 0.25) (layer B.Cu) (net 13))
 (segment (start 154 86) (end 150 86) (width 0.25) (layer B.Cu) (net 13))
 (segment (start 158 90) (end 154 86) (width 0.25) (layer B.Cu) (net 13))
 (segment (start 158 98) (end 158 90) (width 0.25) (layer B.Cu) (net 13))
 (segment (start 156.175 99.825) (end 158 98) (width 0.25) (layer B.Cu) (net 13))
 (segment (start 150 86) (end 150 81.5) (width 0.25) (layer F.Cu) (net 13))
 (segment (start 150.344599 81.337401) (end 150.3976 81.2844) (width 0.25) (layer F.Cu) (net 13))
 (segment (start 158.8392 88.4298) (end 158.8392 86.925228) (width 0.25) (layer F.Cu) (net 11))
 (segment (start 158.8392 86.925228) (end 161.249999 84.514429) (width 0.25) (layer F.Cu) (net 11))
 (segment (start 159.2368 86.709628) (end 161.647599 84.298829) (width 0.25) (layer F.Cu) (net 11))
 (segment (start 154.2 100.475) (end 156.925 100.475) (width 0.25) (layer B.Cu) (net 11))
 (segment (start 158.8368 98.5632) (end 158.8368 88.3142) (width 0.25) (layer B.Cu) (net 11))
 (segment (start 156.925 100.475) (end 158.8368 98.5632) (width 0.25) (layer B.Cu) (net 11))
 (segment (start 134.2012 112.636) (end 133.128429 112.636) (width 0.25) (layer F.Cu) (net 4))
 (segment (start 133.128429 112.636) (end 130.514429 115.25) (width 0.25) (layer F.Cu) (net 4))
 (segment (start 154.2 106.325) (end 155.725 106.325) (width 0.25) (layer B.Cu) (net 4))
 (segment (start 139.0784 117.6) (end 134.0988 112.6204) (width 0.25) (layer B.Cu) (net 4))
 (segment (start 152 117.6) (end 139.0784 117.6) (width 0.25) (layer B.Cu) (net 4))
 (segment (start 157 112.6) (end 152 117.6) (width 0.25) (layer B.Cu) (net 4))
 (segment (start 157 107.6) (end 157 112.6) (width 0.25) (layer B.Cu) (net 4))
 (segment (start 155.725 106.325) (end 157 107.6) (width 0.25) (layer B.Cu) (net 4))
 (segment (start 141.1354 119.494) (end 141.1354 121.100171) (width 0.25) (layer F.Cu) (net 5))
 (segment (start 141.1354 121.100171) (end 138.75 123.485571) (width 0.25) (layer F.Cu) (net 5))
 (segment (start 154.2 105.675) (end 156.075 105.675) (width 0.25) (layer B.Cu) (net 5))
 (segment (start 151.506 119.494) (end 140.8684 119.494) (width 0.25) (layer B.Cu) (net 5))
 (segment (start 157.8 113.2) (end 151.506 119.494) (width 0.25) (layer B.Cu) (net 5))
 (segment (start 157.8 107.4) (end 157.8 113.2) (width 0.25) (layer B.Cu) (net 5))
 (segment (start 156.075 105.675) (end 157.8 107.4) (width 0.25) (layer B.Cu) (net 5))
 (segment (start 150.0762 121.8816) (end 150.0762 126.4238) (width 0.25) (layer F.Cu) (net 6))
 (segment (start 150.0762 126.4238) (end 150 126.5) (width 0.25) (layer F.Cu) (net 6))
 (segment (start 150.4738 126.2082) (end 150.3976 126.2844) (width 0.25) (layer F.Cu) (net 6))
 (segment (start 152.4199 121.9199) (end 150.1145 121.9199) (width 0.25) (layer B.Cu) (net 6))
 (segment (start 150.1145 121.9199) (end 150.0762 121.8816) (width 0.25) (layer B.Cu) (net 6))
 (segment (start 154.2 105.025) (end 156.625 105.025) (width 0.25) (layer B.Cu) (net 6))
 (segment (start 156.625 105.025) (end 158.4 106.8) (width 0.25) (layer B.Cu) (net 6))
 (segment (start 158.4 106.8) (end 158.4 115.9398) (width 0.25) (layer B.Cu) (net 6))
 (segment (start 158.4 115.9398) (end 152.4199 121.9199) (width 0.25) (layer B.Cu) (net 6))
 (segment (start 152.4199 121.9199) (end 152.3738 121.966) (width 0.25) (layer B.Cu) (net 6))
 (segment (start 167.8816 103.9578) (end 172.4578 103.9578) (width 0.25) (layer F.Cu) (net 9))
 (segment (start 172.4578 103.9578) (end 172.5 104) (width 0.25) (layer F.Cu) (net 9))
 (segment (start 172.8554 103.7422) (end 172.8976 103.7844) (width 0.25) (layer F.Cu) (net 9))
 (segment (start 154.2 103.075) (end 167.012 103.075) (width 0.25) (layer B.Cu) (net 9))
 (segment (start 167.012 103.075) (end 167.8792 103.9422) (width 0.25) (layer B.Cu) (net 9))
 (segment (start 158.5852 119.6042) (end 158.5852 120.820772) (width 0.25) (layer F.Cu) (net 7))
 (segment (start 158.5852 120.820772) (end 161.249999 123.485571) (width 0.25) (layer F.Cu) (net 7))
 (segment (start 158.9828 116.6) (end 158.9828 119.2066) (width 0.25) (layer B.Cu) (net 7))
 (segment (start 156.775 104.375) (end 158.9828 106.5828) (width 0.25) (layer B.Cu) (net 7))
 (segment (start 158.9828 106.5828) (end 158.9828 116.6) (width 0.25) (layer B.Cu) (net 7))
 (segment (start 154.2 104.375) (end 156.775 104.375) (width 0.25) (layer B.Cu) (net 7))
 (segment (start 158.9828 119.2066) (end 158.5852 119.6042) (width 0.25) (layer B.Cu) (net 7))
 (segment (start 165.621 112.7716) (end 167.007172 112.7716) (width 0.25) (layer F.Cu) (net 8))
 (segment (start 167.007172 112.7716) (end 169.485571 115.249999) (width 0.25) (layer F.Cu) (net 8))
 (segment (start 167.404772 112.556) (end 169.883171 115.034399) (width 0.25) (layer F.Cu) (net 8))
 (segment (start 164.8186 111.456) (end 164.8186 111.9692) (width 0.25) (layer B.Cu) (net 8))
 (segment (start 157.0876 103.725) (end 164.8186 111.456) (width 0.25) (layer B.Cu) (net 8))
 (segment (start 154.2 103.725) (end 157.0876 103.725) (width 0.25) (layer B.Cu) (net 8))
 (segment (start 164.8186 111.9692) (end 165.621 112.7716) (width 0.25) (layer B.Cu) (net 8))
 (segment (start 154.25 93.5) (end 154.25 96) (width 0.25) (layer B.Cu) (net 19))
 (segment (start 147 107.625) (end 145.668 107.625) (width 0.25) (layer B.Cu) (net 44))
 (segment (start 144.915 108.378) (end 144.0476 108.378) (width 0.25) (layer B.Cu) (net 44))
 (segment (start 145.668 107.625) (end 144.915 108.378) (width 0.25) (layer B.Cu) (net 44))
 (segment (start 147 100.475) (end 144.98 100.475) (width 0.25) (layer B.Cu) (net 48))
 (segment (start 143.311 93.218) (end 144.755 93.218) (width 0.25) (layer B.Cu) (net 48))
 (segment (start 142.676 93.853) (end 143.311 93.218) (width 0.25) (layer B.Cu) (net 48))
 (segment (start 142.676 98.171) (end 142.676 93.853) (width 0.25) (layer B.Cu) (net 48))
 (segment (start 144.98 100.475) (end 142.676 98.171) (width 0.25) (layer B.Cu) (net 48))
 (segment (start 151.75 93.5) (end 147.35 93.5) (width 0.25) (layer B.Cu) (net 22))
 (segment (start 151.75 93.5) (end 151.75 91.1) (width 0.25) (layer B.Cu) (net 22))
 (segment (start 151.75 91.1) (end 151.65 91) (width 0.25) (layer B.Cu) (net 22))
 (segment (start 151.75 96) (end 151.75 93.5) (width 0.25) (layer B.Cu) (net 22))
 (segment (start 148.979 95.758) (end 151.867 95.758) (width 0.25) (layer B.Cu) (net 22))
 (segment (start 154.2 102.425) (end 152.899 102.425) (width 0.25) (layer B.Cu) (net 22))
 (segment (start 151.867 101.393) (end 151.867 95.758) (width 0.25) (layer B.Cu) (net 22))
 (segment (start 152.899 102.425) (end 151.867 101.393) (width 0.25) (layer B.Cu) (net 22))
 (segment (start 144.0476 111.078) (end 148.311 111.078) (width 0.25) (layer B.Cu) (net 22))
 (segment (start 152.9 102.425) (end 154.2 102.425) (width 0.25) (layer B.Cu) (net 22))
 (segment (start 152.074 103.251) (end 152.9 102.425) (width 0.25) (layer B.Cu) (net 22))
 (segment (start 152.074 107.315) (end 152.074 103.251) (width 0.25) (layer B.Cu) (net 22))
 (segment (start 148.311 111.078) (end 152.074 107.315) (width 0.25) (layer B.Cu) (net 22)))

